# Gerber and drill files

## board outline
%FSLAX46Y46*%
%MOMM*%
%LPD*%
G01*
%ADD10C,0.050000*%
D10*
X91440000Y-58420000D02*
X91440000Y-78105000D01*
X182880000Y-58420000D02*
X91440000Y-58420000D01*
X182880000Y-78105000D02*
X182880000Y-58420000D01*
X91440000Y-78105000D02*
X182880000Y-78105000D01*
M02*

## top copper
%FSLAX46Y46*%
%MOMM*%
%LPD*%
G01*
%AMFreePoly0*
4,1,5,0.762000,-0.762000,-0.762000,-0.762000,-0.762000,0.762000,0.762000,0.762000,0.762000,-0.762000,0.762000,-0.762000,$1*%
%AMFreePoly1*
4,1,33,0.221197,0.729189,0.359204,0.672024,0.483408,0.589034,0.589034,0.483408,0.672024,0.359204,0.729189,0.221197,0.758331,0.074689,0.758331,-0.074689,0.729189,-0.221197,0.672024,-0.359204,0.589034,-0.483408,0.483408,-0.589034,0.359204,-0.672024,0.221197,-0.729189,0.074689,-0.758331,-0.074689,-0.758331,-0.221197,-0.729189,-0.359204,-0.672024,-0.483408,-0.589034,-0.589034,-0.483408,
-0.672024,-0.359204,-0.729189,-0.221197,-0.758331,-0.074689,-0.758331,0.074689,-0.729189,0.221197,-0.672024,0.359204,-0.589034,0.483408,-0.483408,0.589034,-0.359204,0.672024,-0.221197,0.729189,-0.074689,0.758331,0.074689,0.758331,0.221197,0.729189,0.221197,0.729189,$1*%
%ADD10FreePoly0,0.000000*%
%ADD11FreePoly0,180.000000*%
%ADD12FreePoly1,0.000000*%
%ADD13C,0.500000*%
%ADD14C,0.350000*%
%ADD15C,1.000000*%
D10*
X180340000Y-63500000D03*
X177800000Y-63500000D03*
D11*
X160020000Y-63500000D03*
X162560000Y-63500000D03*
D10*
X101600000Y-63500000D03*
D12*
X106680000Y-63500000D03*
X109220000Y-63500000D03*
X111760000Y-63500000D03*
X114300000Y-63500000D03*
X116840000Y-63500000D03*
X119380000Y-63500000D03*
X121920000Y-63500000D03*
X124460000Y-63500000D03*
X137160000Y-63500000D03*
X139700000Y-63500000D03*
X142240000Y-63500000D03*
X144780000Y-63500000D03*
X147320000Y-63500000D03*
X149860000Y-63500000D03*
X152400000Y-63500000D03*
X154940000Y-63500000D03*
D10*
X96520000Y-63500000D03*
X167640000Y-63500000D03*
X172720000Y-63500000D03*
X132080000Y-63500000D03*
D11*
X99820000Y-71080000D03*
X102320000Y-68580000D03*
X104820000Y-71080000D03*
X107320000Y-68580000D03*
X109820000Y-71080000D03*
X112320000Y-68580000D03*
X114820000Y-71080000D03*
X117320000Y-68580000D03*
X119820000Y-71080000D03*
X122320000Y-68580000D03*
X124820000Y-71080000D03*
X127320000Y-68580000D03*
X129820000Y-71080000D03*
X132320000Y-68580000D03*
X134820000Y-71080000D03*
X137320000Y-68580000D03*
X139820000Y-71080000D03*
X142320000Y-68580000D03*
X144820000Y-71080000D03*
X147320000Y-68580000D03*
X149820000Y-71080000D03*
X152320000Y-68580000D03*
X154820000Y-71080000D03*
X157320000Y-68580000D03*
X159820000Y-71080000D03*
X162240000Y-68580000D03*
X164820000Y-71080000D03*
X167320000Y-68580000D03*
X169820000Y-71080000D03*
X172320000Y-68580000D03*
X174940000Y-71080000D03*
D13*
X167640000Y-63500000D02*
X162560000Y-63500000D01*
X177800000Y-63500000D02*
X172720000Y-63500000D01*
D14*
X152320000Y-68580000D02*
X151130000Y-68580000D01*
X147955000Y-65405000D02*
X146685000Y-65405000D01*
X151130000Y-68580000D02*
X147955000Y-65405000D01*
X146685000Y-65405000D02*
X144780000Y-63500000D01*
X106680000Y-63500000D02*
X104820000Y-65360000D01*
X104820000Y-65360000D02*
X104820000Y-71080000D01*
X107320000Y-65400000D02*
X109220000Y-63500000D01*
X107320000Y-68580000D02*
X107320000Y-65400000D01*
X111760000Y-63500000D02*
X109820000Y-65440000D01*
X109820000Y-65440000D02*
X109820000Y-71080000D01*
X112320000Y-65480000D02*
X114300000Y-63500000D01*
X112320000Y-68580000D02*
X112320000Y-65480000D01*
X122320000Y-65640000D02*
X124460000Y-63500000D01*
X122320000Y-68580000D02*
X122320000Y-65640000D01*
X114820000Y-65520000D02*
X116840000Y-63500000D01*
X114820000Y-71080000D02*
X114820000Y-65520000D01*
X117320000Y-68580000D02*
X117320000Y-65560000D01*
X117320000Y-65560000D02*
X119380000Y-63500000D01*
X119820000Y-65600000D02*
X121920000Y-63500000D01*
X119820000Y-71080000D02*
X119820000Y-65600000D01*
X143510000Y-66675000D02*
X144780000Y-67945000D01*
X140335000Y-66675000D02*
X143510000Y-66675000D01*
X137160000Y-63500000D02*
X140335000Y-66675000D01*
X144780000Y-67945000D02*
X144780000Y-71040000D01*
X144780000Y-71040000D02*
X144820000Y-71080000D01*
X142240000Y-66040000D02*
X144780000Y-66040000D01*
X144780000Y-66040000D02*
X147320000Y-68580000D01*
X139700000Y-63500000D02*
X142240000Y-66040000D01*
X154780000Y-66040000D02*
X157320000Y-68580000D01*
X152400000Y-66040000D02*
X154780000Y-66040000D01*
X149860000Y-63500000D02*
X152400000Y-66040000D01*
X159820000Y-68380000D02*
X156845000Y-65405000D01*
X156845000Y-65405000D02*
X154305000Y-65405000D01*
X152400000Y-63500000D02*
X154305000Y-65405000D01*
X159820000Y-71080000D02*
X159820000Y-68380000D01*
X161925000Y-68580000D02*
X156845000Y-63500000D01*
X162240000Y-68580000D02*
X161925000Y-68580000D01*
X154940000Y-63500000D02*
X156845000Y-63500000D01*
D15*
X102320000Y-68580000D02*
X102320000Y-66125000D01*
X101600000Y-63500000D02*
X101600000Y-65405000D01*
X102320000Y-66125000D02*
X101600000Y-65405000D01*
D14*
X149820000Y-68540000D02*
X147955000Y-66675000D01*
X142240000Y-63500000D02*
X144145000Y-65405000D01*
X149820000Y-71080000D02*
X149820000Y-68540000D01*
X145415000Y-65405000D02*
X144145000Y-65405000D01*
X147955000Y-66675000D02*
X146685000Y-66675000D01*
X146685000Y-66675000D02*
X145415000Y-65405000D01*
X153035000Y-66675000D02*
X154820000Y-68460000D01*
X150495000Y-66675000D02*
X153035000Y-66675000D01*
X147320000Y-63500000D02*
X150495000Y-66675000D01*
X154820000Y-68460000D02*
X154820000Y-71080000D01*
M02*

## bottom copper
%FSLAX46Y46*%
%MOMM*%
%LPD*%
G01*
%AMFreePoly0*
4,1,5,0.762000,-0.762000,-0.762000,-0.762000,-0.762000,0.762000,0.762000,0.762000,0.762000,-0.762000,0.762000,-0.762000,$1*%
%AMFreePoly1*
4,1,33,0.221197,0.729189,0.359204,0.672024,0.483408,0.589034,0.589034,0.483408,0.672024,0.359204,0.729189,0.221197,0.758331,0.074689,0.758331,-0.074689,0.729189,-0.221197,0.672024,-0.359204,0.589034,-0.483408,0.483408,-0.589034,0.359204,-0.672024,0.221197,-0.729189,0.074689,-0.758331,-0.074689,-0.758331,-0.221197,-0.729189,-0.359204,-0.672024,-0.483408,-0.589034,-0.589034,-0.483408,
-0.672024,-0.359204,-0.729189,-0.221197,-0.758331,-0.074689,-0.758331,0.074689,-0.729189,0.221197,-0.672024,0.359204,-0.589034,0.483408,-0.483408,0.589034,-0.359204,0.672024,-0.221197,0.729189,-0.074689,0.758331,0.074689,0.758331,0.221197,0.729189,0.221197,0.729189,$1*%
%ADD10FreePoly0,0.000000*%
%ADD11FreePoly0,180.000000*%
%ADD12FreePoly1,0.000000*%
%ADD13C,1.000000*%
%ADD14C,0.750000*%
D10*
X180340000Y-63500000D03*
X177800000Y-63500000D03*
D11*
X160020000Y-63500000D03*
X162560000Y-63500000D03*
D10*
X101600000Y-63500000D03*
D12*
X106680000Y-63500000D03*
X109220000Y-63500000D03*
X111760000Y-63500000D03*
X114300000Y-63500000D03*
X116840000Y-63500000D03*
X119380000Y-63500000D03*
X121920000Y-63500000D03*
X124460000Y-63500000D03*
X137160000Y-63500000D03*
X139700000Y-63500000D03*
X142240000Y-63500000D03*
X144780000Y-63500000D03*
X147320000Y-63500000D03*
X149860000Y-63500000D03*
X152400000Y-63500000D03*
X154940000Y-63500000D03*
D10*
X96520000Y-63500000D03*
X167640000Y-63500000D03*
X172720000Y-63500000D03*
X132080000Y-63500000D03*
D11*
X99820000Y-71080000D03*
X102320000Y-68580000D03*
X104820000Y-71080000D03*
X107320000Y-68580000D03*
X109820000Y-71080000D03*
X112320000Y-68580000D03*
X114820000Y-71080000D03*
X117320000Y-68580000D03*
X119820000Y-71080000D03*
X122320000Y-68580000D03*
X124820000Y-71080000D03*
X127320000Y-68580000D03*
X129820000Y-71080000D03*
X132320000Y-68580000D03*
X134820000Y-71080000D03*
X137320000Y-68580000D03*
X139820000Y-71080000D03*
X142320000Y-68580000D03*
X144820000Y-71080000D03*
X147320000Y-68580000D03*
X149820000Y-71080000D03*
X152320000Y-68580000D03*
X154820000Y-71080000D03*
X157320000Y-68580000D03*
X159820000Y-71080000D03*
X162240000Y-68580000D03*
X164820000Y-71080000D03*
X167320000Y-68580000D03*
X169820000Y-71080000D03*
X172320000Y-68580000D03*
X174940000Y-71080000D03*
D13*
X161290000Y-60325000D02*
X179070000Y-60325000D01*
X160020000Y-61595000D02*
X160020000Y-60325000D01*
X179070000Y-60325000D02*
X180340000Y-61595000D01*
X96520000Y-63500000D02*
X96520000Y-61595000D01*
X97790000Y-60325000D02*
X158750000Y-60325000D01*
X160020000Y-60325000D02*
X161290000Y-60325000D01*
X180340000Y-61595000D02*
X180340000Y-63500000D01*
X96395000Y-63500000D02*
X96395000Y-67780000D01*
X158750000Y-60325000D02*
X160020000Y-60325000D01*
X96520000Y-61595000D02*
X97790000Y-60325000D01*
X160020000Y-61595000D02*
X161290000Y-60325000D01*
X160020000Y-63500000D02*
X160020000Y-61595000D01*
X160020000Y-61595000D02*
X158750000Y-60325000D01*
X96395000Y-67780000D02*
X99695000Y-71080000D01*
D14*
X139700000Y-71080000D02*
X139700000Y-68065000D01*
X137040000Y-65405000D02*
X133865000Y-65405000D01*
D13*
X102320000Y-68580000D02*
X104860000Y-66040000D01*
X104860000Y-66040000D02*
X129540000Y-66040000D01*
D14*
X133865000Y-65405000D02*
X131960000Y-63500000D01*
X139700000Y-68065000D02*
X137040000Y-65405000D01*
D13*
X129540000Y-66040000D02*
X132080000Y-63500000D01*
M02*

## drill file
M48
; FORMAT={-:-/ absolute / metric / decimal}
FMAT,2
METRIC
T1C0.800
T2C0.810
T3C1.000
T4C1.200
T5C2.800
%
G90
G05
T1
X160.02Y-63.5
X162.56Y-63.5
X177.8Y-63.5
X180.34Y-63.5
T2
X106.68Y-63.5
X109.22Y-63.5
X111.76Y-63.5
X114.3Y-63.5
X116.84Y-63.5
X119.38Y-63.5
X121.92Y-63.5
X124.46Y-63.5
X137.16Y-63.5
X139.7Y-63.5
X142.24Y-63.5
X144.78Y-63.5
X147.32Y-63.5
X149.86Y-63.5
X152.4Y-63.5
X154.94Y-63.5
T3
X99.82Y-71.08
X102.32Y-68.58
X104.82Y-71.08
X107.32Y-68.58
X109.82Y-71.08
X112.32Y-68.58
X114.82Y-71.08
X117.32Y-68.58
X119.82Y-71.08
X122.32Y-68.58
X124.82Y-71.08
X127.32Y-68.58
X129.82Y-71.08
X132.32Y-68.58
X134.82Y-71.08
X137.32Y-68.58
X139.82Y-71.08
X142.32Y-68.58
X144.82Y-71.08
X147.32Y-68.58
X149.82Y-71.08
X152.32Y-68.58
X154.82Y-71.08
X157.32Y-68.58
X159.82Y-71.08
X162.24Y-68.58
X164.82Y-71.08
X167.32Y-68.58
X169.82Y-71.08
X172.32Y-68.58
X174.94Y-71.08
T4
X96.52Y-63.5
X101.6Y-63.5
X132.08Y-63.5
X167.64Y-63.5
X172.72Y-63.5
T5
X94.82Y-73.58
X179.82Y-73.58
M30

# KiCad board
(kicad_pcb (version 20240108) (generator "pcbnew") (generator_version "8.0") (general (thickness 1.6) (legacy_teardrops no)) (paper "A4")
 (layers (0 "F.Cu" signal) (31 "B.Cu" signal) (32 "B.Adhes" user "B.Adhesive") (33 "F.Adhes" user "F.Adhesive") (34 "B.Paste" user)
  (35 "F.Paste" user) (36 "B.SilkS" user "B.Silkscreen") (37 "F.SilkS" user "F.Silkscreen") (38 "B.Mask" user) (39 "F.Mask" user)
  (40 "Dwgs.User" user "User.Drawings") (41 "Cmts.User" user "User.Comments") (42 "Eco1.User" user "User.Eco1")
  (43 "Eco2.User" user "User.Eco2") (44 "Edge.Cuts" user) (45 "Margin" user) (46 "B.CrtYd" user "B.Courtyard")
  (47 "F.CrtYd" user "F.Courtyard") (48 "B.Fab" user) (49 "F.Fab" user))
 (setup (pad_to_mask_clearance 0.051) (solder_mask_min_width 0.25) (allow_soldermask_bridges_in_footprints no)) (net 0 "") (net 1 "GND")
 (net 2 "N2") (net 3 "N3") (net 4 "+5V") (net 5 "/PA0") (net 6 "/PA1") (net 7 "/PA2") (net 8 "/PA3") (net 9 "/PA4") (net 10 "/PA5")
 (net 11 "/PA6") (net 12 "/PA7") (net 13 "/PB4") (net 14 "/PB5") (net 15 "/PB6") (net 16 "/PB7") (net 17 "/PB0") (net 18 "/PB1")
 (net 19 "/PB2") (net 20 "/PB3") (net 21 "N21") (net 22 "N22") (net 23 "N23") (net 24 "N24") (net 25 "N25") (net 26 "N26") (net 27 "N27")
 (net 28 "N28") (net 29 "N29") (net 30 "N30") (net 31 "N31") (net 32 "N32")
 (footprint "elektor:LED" (layer "F.Cu") (at 177.8 71.12)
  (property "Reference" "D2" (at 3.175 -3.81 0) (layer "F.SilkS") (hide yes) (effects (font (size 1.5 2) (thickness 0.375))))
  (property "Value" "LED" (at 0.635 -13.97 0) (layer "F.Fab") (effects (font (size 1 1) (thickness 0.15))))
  (pad "1" thru_hole custom (at 2.54 -7.62) (size 1.524 1.524) (drill 0.8) (layers "*.Cu" "*.Mask") (remove_unused_layers no) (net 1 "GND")
   (zone_connect 0) (thermal_bridge_angle 45) (options (clearance outline) (anchor rect)) (primitives))
  (pad "2" thru_hole custom (at 0 -7.62) (size 1.524 1.524) (drill 0.8) (layers "*.Cu" "*.Mask") (remove_unused_layers no) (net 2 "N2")
   (zone_connect 0) (thermal_bridge_angle 45) (options (clearance outline) (anchor rect)) (primitives)))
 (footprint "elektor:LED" (layer "F.Cu") (at 162.56 55.88 180)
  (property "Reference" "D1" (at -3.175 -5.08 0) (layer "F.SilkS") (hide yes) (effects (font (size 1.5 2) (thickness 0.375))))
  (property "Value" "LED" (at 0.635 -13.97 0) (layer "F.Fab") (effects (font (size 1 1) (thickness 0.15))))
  (pad "1" thru_hole custom (at 2.54 -7.62 180) (size 1.524 1.524) (drill 0.8) (layers "*.Cu" "*.Mask") (remove_unused_layers no)
   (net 1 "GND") (zone_connect 0) (thermal_bridge_angle 45) (options (clearance outline) (anchor rect)) (primitives))
  (pad "2" thru_hole custom (at 0 -7.62 180) (size 1.524 1.524) (drill 0.8) (layers "*.Cu" "*.Mask") (remove_unused_layers no) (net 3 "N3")
   (zone_connect 0) (thermal_bridge_angle 45) (options (clearance outline) (anchor rect)) (primitives)))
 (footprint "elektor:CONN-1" (layer "F.Cu") (at 101.6 63.5)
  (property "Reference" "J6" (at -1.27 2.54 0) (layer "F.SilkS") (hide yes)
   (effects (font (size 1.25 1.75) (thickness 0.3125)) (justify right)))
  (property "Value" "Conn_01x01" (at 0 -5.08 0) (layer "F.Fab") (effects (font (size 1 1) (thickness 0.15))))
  (pad "1" thru_hole custom (at 0 0) (size 1.524 1.524) (drill 1.2) (layers "*.Cu" "*.Mask") (remove_unused_layers no) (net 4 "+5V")
   (zone_connect 0) (thermal_bridge_angle 45) (options (clearance outline) (anchor rect)) (primitives)))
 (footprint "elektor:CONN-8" (layer "F.Cu") (at 109.22 63.5)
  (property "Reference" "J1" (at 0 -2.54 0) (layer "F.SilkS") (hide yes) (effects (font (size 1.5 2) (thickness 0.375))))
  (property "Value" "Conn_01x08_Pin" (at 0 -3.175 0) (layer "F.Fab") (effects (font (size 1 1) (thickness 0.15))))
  (pad "1" thru_hole custom (at -2.54 0) (size 1.524 1.524) (drill 0.81) (layers "*.Cu" "*.Mask") (remove_unused_layers no) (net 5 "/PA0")
   (zone_connect 0) (options (clearance outline) (anchor circle)) (primitives))
  (pad "2" thru_hole custom (at 0 0) (size 1.524 1.524) (drill 0.81) (layers "*.Cu" "*.Mask") (remove_unused_layers no) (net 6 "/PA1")
   (zone_connect 0) (options (clearance outline) (anchor circle)) (primitives))
  (pad "3" thru_hole custom (at 2.54 0) (size 1.524 1.524) (drill 0.81) (layers "*.Cu" "*.Mask") (remove_unused_layers no) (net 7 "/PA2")
   (zone_connect 0) (options (clearance outline) (anchor circle)) (primitives))
  (pad "4" thru_hole custom (at 5.08 0) (size 1.524 1.524) (drill 0.81) (layers "*.Cu" "*.Mask") (remove_unused_layers no) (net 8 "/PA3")
   (zone_connect 0) (options (clearance outline) (anchor circle)) (primitives))
  (pad "5" thru_hole custom (at 7.62 0) (size 1.524 1.524) (drill 0.81) (layers "*.Cu" "*.Mask") (remove_unused_layers no) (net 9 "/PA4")
   (zone_connect 0) (options (clearance outline) (anchor circle)) (primitives))
  (pad "6" thru_hole custom (at 10.16 0) (size 1.524 1.524) (drill 0.81) (layers "*.Cu" "*.Mask") (remove_unused_layers no) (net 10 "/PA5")
   (zone_connect 0) (options (clearance outline) (anchor circle)) (primitives))
  (pad "7" thru_hole custom (at 12.7 0) (size 1.524 1.524) (drill 0.81) (layers "*.Cu" "*.Mask") (remove_unused_layers no) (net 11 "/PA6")
   (zone_connect 0) (options (clearance outline) (anchor circle)) (primitives))
  (pad "8" thru_hole custom (at 15.24 0) (size 1.524 1.524) (drill 0.81) (layers "*.Cu" "*.Mask") (remove_unused_layers no) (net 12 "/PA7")
   (zone_connect 0) (options (clearance outline) (anchor circle)) (primitives)))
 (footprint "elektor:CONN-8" (layer "F.Cu") (at 139.7 63.5)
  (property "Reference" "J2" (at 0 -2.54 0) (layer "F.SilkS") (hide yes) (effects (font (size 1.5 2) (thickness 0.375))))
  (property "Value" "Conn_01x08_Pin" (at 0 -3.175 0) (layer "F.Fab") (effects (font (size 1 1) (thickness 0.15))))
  (pad "1" thru_hole custom (at -2.54 0) (size 1.524 1.524) (drill 0.81) (layers "*.Cu" "*.Mask") (remove_unused_layers no) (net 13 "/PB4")
   (zone_connect 0) (options (clearance outline) (anchor circle)) (primitives))
  (pad "2" thru_hole custom (at 0 0) (size 1.524 1.524) (drill 0.81) (layers "*.Cu" "*.Mask") (remove_unused_layers no) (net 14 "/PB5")
   (zone_connect 0) (options (clearance outline) (anchor circle)) (primitives))
  (pad "3" thru_hole custom (at 2.54 0) (size 1.524 1.524) (drill 0.81) (layers "*.Cu" "*.Mask") (remove_unused_layers no) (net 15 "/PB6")
   (zone_connect 0) (options (clearance outline) (anchor circle)) (primitives))
  (pad "4" thru_hole custom (at 5.08 0) (size 1.524 1.524) (drill 0.81) (layers "*.Cu" "*.Mask") (remove_unused_layers no) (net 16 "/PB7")
   (zone_connect 0) (options (clearance outline) (anchor circle)) (primitives))
  (pad "5" thru_hole custom (at 7.62 0) (size 1.524 1.524) (drill 0.81) (layers "*.Cu" "*.Mask") (remove_unused_layers no) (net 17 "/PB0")
   (zone_connect 0) (options (clearance outline) (anchor circle)) (primitives))
  (pad "6" thru_hole custom (at 10.16 0) (size 1.524 1.524) (drill 0.81) (layers "*.Cu" "*.Mask") (remove_unused_layers no) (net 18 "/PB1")
   (zone_connect 0) (options (clearance outline) (anchor circle)) (primitives))
  (pad "7" thru_hole custom (at 12.7 0) (size 1.524 1.524) (drill 0.81) (layers "*.Cu" "*.Mask") (remove_unused_layers no) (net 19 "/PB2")
   (zone_connect 0) (options (clearance outline) (anchor circle)) (primitives))
  (pad "8" thru_hole custom (at 15.24 0) (size 1.524 1.524) (drill 0.81) (layers "*.Cu" "*.Mask") (remove_unused_layers no) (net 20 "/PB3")
   (zone_connect 0) (options (clearance outline) (anchor circle)) (primitives)))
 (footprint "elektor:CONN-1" (layer "F.Cu") (at 96.52 63.5)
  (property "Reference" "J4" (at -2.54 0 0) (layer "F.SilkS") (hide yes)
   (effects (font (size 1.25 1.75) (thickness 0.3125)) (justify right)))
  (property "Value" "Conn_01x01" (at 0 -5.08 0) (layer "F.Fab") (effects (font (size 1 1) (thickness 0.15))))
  (pad "1" thru_hole custom (at 0 0) (size 1.524 1.524) (drill 1.2) (layers "*.Cu" "*.Mask") (remove_unused_layers no) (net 1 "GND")
   (zone_connect 0) (thermal_bridge_angle 45) (options (clearance outline) (anchor rect)) (primitives)))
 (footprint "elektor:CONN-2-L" (layer "F.Cu") (at 172.72 63.5)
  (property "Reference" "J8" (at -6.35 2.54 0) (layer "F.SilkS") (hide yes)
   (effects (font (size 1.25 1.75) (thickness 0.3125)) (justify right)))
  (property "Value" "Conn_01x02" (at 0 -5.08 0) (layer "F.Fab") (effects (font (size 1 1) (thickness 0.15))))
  (pad "1" thru_hole custom (at -5.08 0) (size 1.524 1.524) (drill 1.2) (layers "*.Cu" "*.Mask") (remove_unused_layers no) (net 3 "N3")
   (zone_connect 0) (thermal_bridge_angle 45) (options (clearance outline) (anchor rect)) (primitives))
  (pad "2" thru_hole custom (at 0 0) (size 1.524 1.524) (drill 1.2) (layers "*.Cu" "*.Mask") (remove_unused_layers no) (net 2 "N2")
   (zone_connect 0) (thermal_bridge_angle 45) (options (clearance outline) (anchor rect)) (primitives)))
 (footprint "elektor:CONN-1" (layer "F.Cu") (at 132.08 63.5)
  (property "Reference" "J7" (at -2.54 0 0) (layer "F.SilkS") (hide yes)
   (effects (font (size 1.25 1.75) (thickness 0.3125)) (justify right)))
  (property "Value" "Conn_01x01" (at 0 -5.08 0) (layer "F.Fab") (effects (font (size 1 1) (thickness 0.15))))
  (pad "1" thru_hole custom (at 0 0) (size 1.524 1.524) (drill 1.2) (layers "*.Cu" "*.Mask") (remove_unused_layers no) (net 4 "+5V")
   (zone_connect 0) (thermal_bridge_angle 45) (options (clearance outline) (anchor rect)) (primitives)))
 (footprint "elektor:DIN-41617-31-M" (layer "B.Cu") (at 167.32 66.08 180)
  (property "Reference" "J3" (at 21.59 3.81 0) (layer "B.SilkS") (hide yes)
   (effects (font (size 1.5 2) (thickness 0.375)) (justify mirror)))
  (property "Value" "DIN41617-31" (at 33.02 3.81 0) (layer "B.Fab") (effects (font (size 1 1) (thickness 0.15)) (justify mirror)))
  (pad "" np_thru_hole circle (at -12.5 -7.5 180) (size 2.8 2.8) (drill 2.8) (layers "*.Cu" "*.Mask") (zone_connect 0))
  (pad "" np_thru_hole circle (at 72.5 -7.5 180) (size 2.8 2.8) (drill 2.8) (layers "*.Cu" "*.Mask") (zone_connect 0))
  (pad "1" thru_hole custom (at 67.5 -5 180) (size 1.524 1.524) (drill 1) (layers "*.Cu" "*.Mask") (remove_unused_layers no) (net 1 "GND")
   (zone_connect 0) (thermal_bridge_angle 45) (options (clearance outline) (anchor rect)) (primitives))
  (pad "2" thru_hole custom (at 65 -2.5 180) (size 1.524 1.524) (drill 1) (layers "*.Cu" "*.Mask") (remove_unused_layers no) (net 4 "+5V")
   (zone_connect 0) (thermal_bridge_angle 45) (options (clearance outline) (anchor rect)) (primitives))
  (pad "3" thru_hole custom (at 62.5 -5 180) (size 1.524 1.524) (drill 1) (layers "*.Cu" "*.Mask") (remove_unused_layers no) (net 5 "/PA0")
   (zone_connect 0) (thermal_bridge_angle 45) (options (clearance outline) (anchor rect)) (primitives))
  (pad "4" thru_hole custom (at 60 -2.5 180) (size 1.524 1.524) (drill 1) (layers "*.Cu" "*.Mask") (remove_unused_layers no) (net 6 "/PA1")
   (zone_connect 0) (thermal_bridge_angle 45) (options (clearance outline) (anchor rect)) (primitives))
  (pad "5" thru_hole custom (at 57.5 -5 180) (size 1.524 1.524) (drill 1) (layers "*.Cu" "*.Mask") (remove_unused_layers no) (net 7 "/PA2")
   (zone_connect 0) (thermal_bridge_angle 45) (options (clearance outline) (anchor rect)) (primitives))
  (pad "6" thru_hole custom (at 55 -2.5 180) (size 1.524 1.524) (drill 1) (layers "*.Cu" "*.Mask") (remove_unused_layers no) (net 8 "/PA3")
   (zone_connect 0) (thermal_bridge_angle 45) (options (clearance outline) (anchor rect)) (primitives))
  (pad "7" thru_hole custom (at 52.5 -5 180) (size 1.524 1.524) (drill 1) (layers "*.Cu" "*.Mask") (remove_unused_layers no) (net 9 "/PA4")
   (zone_connect 0) (thermal_bridge_angle 45) (options (clearance outline) (anchor rect)) (primitives))
  (pad "8" thru_hole custom (at 50 -2.5 180) (size 1.524 1.524) (drill 1) (layers "*.Cu" "*.Mask") (remove_unused_layers no) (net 10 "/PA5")
   (zone_connect 0) (thermal_bridge_angle 45) (options (clearance outline) (anchor rect)) (primitives))
  (pad "9" thru_hole custom (at 47.5 -5 180) (size 1.524 1.524) (drill 1) (layers "*.Cu" "*.Mask") (remove_unused_layers no) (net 11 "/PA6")
   (zone_connect 0) (thermal_bridge_angle 45) (options (clearance outline) (anchor rect)) (primitives))
  (pad "10" thru_hole custom (at 45 -2.5 180) (size 1.524 1.524) (drill 1) (layers "*.Cu" "*.Mask") (remove_unused_layers no)
   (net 12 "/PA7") (zone_connect 0) (thermal_bridge_angle 45) (options (clearance outline) (anchor rect)) (primitives))
  (pad "11" thru_hole custom (at 42.5 -5 180) (size 1.524 1.524) (drill 1) (layers "*.Cu" "*.Mask") (remove_unused_layers no) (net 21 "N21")
   (zone_connect 0) (thermal_bridge_angle 45) (options (clearance outline) (anchor rect)) (primitives))
  (pad "12" thru_hole custom (at 40 -2.5 180) (size 1.524 1.524) (drill 1) (layers "*.Cu" "*.Mask") (remove_unused_layers no) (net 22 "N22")
   (zone_connect 0) (thermal_bridge_angle 45) (options (clearance outline) (anchor rect)) (primitives))
  (pad "13" thru_hole custom (at 37.5 -5 180) (size 1.524 1.524) (drill 1) (layers "*.Cu" "*.Mask") (remove_unused_layers no) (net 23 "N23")
   (zone_connect 0) (thermal_bridge_angle 45) (options (clearance outline) (anchor rect)) (primitives))
  (pad "14" thru_hole custom (at 35 -2.5 180) (size 1.524 1.524) (drill 1) (layers "*.Cu" "*.Mask") (remove_unused_layers no) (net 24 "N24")
   (zone_connect 0) (thermal_bridge_angle 45) (options (clearance outline) (anchor rect)) (primitives))
  (pad "15" thru_hole custom (at 32.5 -5 180) (size 1.524 1.524) (drill 1) (layers "*.Cu" "*.Mask") (remove_unused_layers no) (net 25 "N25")
   (zone_connect 0) (thermal_bridge_angle 45) (options (clearance outline) (anchor rect)) (primitives))
  (pad "16" thru_hole custom (at 30 -2.5 180) (size 1.524 1.524) (drill 1) (layers "*.Cu" "*.Mask") (remove_unused_layers no) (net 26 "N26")
   (zone_connect 0) (thermal_bridge_angle 45) (options (clearance outline) (anchor rect)) (primitives))
  (pad "17" thru_hole custom (at 27.5 -5 180) (size 1.524 1.524) (drill 1) (layers "*.Cu" "*.Mask") (remove_unused_layers no) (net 4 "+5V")
   (zone_connect 0) (thermal_bridge_angle 45) (options (clearance outline) (anchor rect)) (primitives))
  (pad "18" thru_hole custom (at 25 -2.5 180) (size 1.524 1.524) (drill 1) (layers "*.Cu" "*.Mask") (remove_unused_layers no) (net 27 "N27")
   (zone_connect 0) (thermal_bridge_angle 45) (options (clearance outline) (anchor rect)) (primitives))
  (pad "19" thru_hole custom (at 22.5 -5 180) (size 1.524 1.524) (drill 1) (layers "*.Cu" "*.Mask") (remove_unused_layers no)
   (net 13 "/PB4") (zone_connect 0) (thermal_bridge_angle 45) (options (clearance outline) (anchor rect)) (primitives))
  (pad "20" thru_hole custom (at 20 -2.5 180) (size 1.524 1.524) (drill 1) (layers "*.Cu" "*.Mask") (remove_unused_layers no)
   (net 14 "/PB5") (zone_connect 0) (thermal_bridge_angle 45) (options (clearance outline) (anchor rect)) (primitives))
  (pad "21" thru_hole custom (at 17.5 -5 180) (size 1.524 1.524) (drill 1) (layers "*.Cu" "*.Mask") (remove_unused_layers no)
   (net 15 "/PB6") (zone_connect 0) (thermal_bridge_angle 45) (options (clearance outline) (anchor rect)) (primitives))
  (pad "22" thru_hole custom (at 15 -2.5 180) (size 1.524 1.524) (drill 1) (layers "*.Cu" "*.Mask") (remove_unused_layers no)
   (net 16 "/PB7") (zone_connect 0) (thermal_bridge_angle 45) (options (clearance outline) (anchor rect)) (primitives))
  (pad "23" thru_hole custom (at 12.5 -5 180) (size 1.524 1.524) (drill 1) (layers "*.Cu" "*.Mask") (remove_unused_layers no)
   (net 17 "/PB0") (zone_connect 0) (thermal_bridge_angle 45) (options (clearance outline) (anchor rect)) (primitives))
  (pad "24" thru_hole custom (at 10 -2.5 180) (size 1.524 1.524) (drill 1) (layers "*.Cu" "*.Mask") (remove_unused_layers no)
   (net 18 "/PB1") (zone_connect 0) (thermal_bridge_angle 45) (options (clearance outline) (anchor rect)) (primitives))
  (pad "25" thru_hole custom (at 7.5 -5 180) (size 1.524 1.524) (drill 1) (layers "*.Cu" "*.Mask") (remove_unused_layers no) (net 19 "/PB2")
   (zone_connect 0) (thermal_bridge_angle 45) (options (clearance outline) (anchor rect)) (primitives))
  (pad "26" thru_hole custom (at 5.08 -2.5 180) (size 1.524 1.524) (drill 1) (layers "*.Cu" "*.Mask") (remove_unused_layers no)
   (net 20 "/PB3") (zone_connect 0) (thermal_bridge_angle 45) (options (clearance outline) (anchor rect)) (primitives))
  (pad "27" thru_hole custom (at 2.5 -5 180) (size 1.524 1.524) (drill 1) (layers "*.Cu" "*.Mask") (remove_unused_layers no) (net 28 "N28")
   (zone_connect 0) (thermal_bridge_angle 45) (options (clearance outline) (anchor rect)) (primitives))
  (pad "28" thru_hole custom (at 0 -2.5 180) (size 1.524 1.524) (drill 1) (layers "*.Cu" "*.Mask") (remove_unused_layers no) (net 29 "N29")
   (zone_connect 0) (thermal_bridge_angle 45) (options (clearance outline) (anchor rect)) (primitives))
  (pad "29" thru_hole custom (at -2.5 -5 180) (size 1.524 1.524) (drill 1) (layers "*.Cu" "*.Mask") (remove_unused_layers no) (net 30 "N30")
   (zone_connect 0) (thermal_bridge_angle 45) (options (clearance outline) (anchor rect)) (primitives))
  (pad "30" thru_hole custom (at -5 -2.5 180) (size 1.524 1.524) (drill 1) (layers "*.Cu" "*.Mask") (remove_unused_layers no) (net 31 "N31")
   (zone_connect 0) (thermal_bridge_angle 45) (options (clearance outline) (anchor rect)) (primitives))
  (pad "31" thru_hole custom (at -7.62 -5 180) (size 1.524 1.524) (drill 1) (layers "*.Cu" "*.Mask") (remove_unused_layers no)
   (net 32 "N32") (zone_connect 0) (thermal_bridge_angle 45) (options (clearance outline) (anchor rect)) (primitives)))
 (gr_line (start 91.44 58.42) (end 91.44 78.105) (stroke (width 0.05) (type solid)) (layer "Edge.Cuts"))
 (gr_line (start 182.88 58.42) (end 91.44 58.42) (stroke (width 0.05) (type solid)) (layer "Edge.Cuts"))
 (gr_line (start 182.88 78.105) (end 182.88 58.42) (stroke (width 0.05) (type solid)) (layer "Edge.Cuts"))
 (gr_line (start 91.44 78.105) (end 182.88 78.105) (stroke (width 0.05) (type solid)) (layer "Edge.Cuts"))
 (segment (start 167.64 63.5) (end 162.56 63.5) (width 0.5) (layer "F.Cu") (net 3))
 (segment (start 161.29 60.325) (end 179.07 60.325) (width 1) (layer "B.Cu") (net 1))
 (segment (start 160.02 61.595) (end 160.02 60.325) (width 1) (layer "B.Cu") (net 1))
 (segment (start 179.07 60.325) (end 180.34 61.595) (width 1) (layer "B.Cu") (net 1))
 (segment (start 96.52 63.5) (end 96.52 61.595) (width 1) (layer "B.Cu") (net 1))
 (segment (start 97.79 60.325) (end 158.75 60.325) (width 1) (layer "B.Cu") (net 1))
 (segment (start 160.02 60.325) (end 161.29 60.325) (width 1) (layer "B.Cu") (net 1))
 (segment (start 180.34 61.595) (end 180.34 63.5) (width 1) (layer "B.Cu") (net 1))
 (segment (start 96.395 63.5) (end 96.395 67.78) (width 1) (layer "B.Cu") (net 1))
 (segment (start 158.75 60.325) (end 160.02 60.325) (width 1) (layer "B.Cu") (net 1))
 (segment (start 96.52 61.595) (end 97.79 60.325) (width 1) (layer "B.Cu") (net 1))
 (segment (start 160.02 61.595) (end 161.29 60.325) (width 1) (layer "B.Cu") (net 1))
 (segment (start 160.02 63.5) (end 160.02 61.595) (width 1) (layer "B.Cu") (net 1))
 (segment (start 160.02 61.595) (end 158.75 60.325) (width 1) (layer "B.Cu") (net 1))
 (segment (start 96.395 67.78) (end 99.695 71.08) (width 1) (layer "B.Cu") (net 1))
 (segment (start 177.8 63.5) (end 172.72 63.5) (width 0.5) (layer "F.Cu") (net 2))
 (segment (start 152.32 68.58) (end 151.13 68.58) (width 0.35) (layer "F.Cu") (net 16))
 (segment (start 147.955 65.405) (end 146.685 65.405) (width 0.35) (layer "F.Cu") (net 16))
 (segment (start 151.13 68.58) (end 147.955 65.405) (width 0.35) (layer "F.Cu") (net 16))
 (segment (start 146.685 65.405) (end 144.78 63.5) (width 0.35) (layer "F.Cu") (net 16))
 (segment (start 106.68 63.5) (end 104.82 65.36) (width 0.35) (layer "F.Cu") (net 5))
 (segment (start 104.82 65.36) (end 104.82 71.08) (width 0.35) (layer "F.Cu") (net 5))
 (segment (start 107.32 65.4) (end 109.22 63.5) (width 0.35) (layer "F.Cu") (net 6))
 (segment (start 107.32 68.58) (end 107.32 65.4) (width 0.35) (layer "F.Cu") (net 6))
 (segment (start 111.76 63.5) (end 109.82 65.44) (width 0.35) (layer "F.Cu") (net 7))
 (segment (start 109.82 65.44) (end 109.82 71.08) (width 0.35) (layer "F.Cu") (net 7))
 (segment (start 112.32 65.48) (end 114.3 63.5) (width 0.35) (layer "F.Cu") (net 8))
 (segment (start 112.32 68.58) (end 112.32 65.48) (width 0.35) (layer "F.Cu") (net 8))
 (segment (start 122.32 65.64) (end 124.46 63.5) (width 0.35) (layer "F.Cu") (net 12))
 (segment (start 122.32 68.58) (end 122.32 65.64) (width 0.35) (layer "F.Cu") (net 12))
 (segment (start 114.82 65.52) (end 116.84 63.5) (width 0.35) (layer "F.Cu") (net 9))
 (segment (start 114.82 71.08) (end 114.82 65.52) (width 0.35) (layer "F.Cu") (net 9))
 (segment (start 117.32 68.58) (end 117.32 65.56) (width 0.35) (layer "F.Cu") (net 10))
 (segment (start 117.32 65.56) (end 119.38 63.5) (width 0.35) (layer "F.Cu") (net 10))
 (segment (start 119.82 65.6) (end 121.92 63.5) (width 0.35) (layer "F.Cu") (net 11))
 (segment (start 119.82 71.08) (end 119.82 65.6) (width 0.35) (layer "F.Cu") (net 11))
 (segment (start 143.51 66.675) (end 144.78 67.945) (width 0.35) (layer "F.Cu") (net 13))
 (segment (start 140.335 66.675) (end 143.51 66.675) (width 0.35) (layer "F.Cu") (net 13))
 (segment (start 137.16 63.5) (end 140.335 66.675) (width 0.35) (layer "F.Cu") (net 13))
 (segment (start 144.78 67.945) (end 144.78 71.04) (width 0.35) (layer "F.Cu") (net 13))
 (segment (start 144.78 71.04) (end 144.82 71.08) (width 0.35) (layer "F.Cu") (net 13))
 (segment (start 142.24 66.04) (end 144.78 66.04) (width 0.35) (layer "F.Cu") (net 14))
 (segment (start 144.78 66.04) (end 147.32 68.58) (width 0.35) (layer "F.Cu") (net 14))
 (segment (start 139.7 63.5) (end 142.24 66.04) (width 0.35) (layer "F.Cu") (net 14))
 (segment (start 154.78 66.04) (end 157.32 68.58) (width 0.35) (layer "F.Cu") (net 18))
 (segment (start 152.4 66.04) (end 154.78 66.04) (width 0.35) (layer "F.Cu") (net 18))
 (segment (start 149.86 63.5) (end 152.4 66.04) (width 0.35) (layer "F.Cu") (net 18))
 (segment (start 159.82 68.38) (end 156.845 65.405) (width 0.35) (layer "F.Cu") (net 19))
 (segment (start 156.845 65.405) (end 154.305 65.405) (width 0.35) (layer "F.Cu") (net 19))
 (segment (start 152.4 63.5) (end 154.305 65.405) (width 0.35) (layer "F.Cu") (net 19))
 (segment (start 159.82 71.08) (end 159.82 68.38) (width 0.35) (layer "F.Cu") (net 19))
 (segment (start 161.925 68.58) (end 156.845 63.5) (width 0.35) (layer "F.Cu") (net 20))
 (segment (start 162.24 68.58) (end 161.925 68.58) (width 0.35) (layer "F.Cu") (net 20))
 (segment (start 154.94 63.5) (end 156.845 63.5) (width 0.35) (layer "F.Cu") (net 20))
 (segment (start 102.32 68.58) (end 102.32 66.125) (width 1) (layer "F.Cu") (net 4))
 (segment (start 101.6 63.5) (end 101.6 65.405) (width 1) (layer "F.Cu") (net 4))
 (segment (start 102.32 66.125) (end 101.6 65.405) (width 1) (layer "F.Cu") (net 4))
 (segment (start 139.7 71.08) (end 139.7 68.065) (width 0.75) (layer "B.Cu") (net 4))
 (segment (start 137.04 65.405) (end 133.865 65.405) (width 0.75) (layer "B.Cu") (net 4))
 (segment (start 102.32 68.58) (end 104.86 66.04) (width 1) (layer "B.Cu") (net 4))
 (segment (start 104.86 66.04) (end 129.54 66.04) (width 1) (layer "B.Cu") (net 4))
 (segment (start 133.865 65.405) (end 131.96 63.5) (width 0.75) (layer "B.Cu") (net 4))
 (segment (start 139.7 68.065) (end 137.04 65.405) (width 0.75) (layer "B.Cu") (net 4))
 (segment (start 129.54 66.04) (end 132.08 63.5) (width 1) (layer "B.Cu") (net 4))
 (segment (start 149.82 68.54) (end 147.955 66.675) (width 0.35) (layer "F.Cu") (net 15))
 (segment (start 142.24 63.5) (end 144.145 65.405) (width 0.35) (layer "F.Cu") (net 15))
 (segment (start 149.82 71.08) (end 149.82 68.54) (width 0.35) (layer "F.Cu") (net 15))
 (segment (start 145.415 65.405) (end 144.145 65.405) (width 0.35) (layer "F.Cu") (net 15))
 (segment (start 147.955 66.675) (end 146.685 66.675) (width 0.35) (layer "F.Cu") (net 15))
 (segment (start 146.685 66.675) (end 145.415 65.405) (width 0.35) (layer "F.Cu") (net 15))
 (segment (start 153.035 66.675) (end 154.82 68.46) (width 0.35) (layer "F.Cu") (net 17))
 (segment (start 150.495 66.675) (end 153.035 66.675) (width 0.35) (layer "F.Cu") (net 17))
 (segment (start 147.32 63.5) (end 150.495 66.675) (width 0.35) (layer "F.Cu") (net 17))
 (segment (start 154.82 68.46) (end 154.82 71.08) (width 0.35) (layer "F.Cu") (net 17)))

